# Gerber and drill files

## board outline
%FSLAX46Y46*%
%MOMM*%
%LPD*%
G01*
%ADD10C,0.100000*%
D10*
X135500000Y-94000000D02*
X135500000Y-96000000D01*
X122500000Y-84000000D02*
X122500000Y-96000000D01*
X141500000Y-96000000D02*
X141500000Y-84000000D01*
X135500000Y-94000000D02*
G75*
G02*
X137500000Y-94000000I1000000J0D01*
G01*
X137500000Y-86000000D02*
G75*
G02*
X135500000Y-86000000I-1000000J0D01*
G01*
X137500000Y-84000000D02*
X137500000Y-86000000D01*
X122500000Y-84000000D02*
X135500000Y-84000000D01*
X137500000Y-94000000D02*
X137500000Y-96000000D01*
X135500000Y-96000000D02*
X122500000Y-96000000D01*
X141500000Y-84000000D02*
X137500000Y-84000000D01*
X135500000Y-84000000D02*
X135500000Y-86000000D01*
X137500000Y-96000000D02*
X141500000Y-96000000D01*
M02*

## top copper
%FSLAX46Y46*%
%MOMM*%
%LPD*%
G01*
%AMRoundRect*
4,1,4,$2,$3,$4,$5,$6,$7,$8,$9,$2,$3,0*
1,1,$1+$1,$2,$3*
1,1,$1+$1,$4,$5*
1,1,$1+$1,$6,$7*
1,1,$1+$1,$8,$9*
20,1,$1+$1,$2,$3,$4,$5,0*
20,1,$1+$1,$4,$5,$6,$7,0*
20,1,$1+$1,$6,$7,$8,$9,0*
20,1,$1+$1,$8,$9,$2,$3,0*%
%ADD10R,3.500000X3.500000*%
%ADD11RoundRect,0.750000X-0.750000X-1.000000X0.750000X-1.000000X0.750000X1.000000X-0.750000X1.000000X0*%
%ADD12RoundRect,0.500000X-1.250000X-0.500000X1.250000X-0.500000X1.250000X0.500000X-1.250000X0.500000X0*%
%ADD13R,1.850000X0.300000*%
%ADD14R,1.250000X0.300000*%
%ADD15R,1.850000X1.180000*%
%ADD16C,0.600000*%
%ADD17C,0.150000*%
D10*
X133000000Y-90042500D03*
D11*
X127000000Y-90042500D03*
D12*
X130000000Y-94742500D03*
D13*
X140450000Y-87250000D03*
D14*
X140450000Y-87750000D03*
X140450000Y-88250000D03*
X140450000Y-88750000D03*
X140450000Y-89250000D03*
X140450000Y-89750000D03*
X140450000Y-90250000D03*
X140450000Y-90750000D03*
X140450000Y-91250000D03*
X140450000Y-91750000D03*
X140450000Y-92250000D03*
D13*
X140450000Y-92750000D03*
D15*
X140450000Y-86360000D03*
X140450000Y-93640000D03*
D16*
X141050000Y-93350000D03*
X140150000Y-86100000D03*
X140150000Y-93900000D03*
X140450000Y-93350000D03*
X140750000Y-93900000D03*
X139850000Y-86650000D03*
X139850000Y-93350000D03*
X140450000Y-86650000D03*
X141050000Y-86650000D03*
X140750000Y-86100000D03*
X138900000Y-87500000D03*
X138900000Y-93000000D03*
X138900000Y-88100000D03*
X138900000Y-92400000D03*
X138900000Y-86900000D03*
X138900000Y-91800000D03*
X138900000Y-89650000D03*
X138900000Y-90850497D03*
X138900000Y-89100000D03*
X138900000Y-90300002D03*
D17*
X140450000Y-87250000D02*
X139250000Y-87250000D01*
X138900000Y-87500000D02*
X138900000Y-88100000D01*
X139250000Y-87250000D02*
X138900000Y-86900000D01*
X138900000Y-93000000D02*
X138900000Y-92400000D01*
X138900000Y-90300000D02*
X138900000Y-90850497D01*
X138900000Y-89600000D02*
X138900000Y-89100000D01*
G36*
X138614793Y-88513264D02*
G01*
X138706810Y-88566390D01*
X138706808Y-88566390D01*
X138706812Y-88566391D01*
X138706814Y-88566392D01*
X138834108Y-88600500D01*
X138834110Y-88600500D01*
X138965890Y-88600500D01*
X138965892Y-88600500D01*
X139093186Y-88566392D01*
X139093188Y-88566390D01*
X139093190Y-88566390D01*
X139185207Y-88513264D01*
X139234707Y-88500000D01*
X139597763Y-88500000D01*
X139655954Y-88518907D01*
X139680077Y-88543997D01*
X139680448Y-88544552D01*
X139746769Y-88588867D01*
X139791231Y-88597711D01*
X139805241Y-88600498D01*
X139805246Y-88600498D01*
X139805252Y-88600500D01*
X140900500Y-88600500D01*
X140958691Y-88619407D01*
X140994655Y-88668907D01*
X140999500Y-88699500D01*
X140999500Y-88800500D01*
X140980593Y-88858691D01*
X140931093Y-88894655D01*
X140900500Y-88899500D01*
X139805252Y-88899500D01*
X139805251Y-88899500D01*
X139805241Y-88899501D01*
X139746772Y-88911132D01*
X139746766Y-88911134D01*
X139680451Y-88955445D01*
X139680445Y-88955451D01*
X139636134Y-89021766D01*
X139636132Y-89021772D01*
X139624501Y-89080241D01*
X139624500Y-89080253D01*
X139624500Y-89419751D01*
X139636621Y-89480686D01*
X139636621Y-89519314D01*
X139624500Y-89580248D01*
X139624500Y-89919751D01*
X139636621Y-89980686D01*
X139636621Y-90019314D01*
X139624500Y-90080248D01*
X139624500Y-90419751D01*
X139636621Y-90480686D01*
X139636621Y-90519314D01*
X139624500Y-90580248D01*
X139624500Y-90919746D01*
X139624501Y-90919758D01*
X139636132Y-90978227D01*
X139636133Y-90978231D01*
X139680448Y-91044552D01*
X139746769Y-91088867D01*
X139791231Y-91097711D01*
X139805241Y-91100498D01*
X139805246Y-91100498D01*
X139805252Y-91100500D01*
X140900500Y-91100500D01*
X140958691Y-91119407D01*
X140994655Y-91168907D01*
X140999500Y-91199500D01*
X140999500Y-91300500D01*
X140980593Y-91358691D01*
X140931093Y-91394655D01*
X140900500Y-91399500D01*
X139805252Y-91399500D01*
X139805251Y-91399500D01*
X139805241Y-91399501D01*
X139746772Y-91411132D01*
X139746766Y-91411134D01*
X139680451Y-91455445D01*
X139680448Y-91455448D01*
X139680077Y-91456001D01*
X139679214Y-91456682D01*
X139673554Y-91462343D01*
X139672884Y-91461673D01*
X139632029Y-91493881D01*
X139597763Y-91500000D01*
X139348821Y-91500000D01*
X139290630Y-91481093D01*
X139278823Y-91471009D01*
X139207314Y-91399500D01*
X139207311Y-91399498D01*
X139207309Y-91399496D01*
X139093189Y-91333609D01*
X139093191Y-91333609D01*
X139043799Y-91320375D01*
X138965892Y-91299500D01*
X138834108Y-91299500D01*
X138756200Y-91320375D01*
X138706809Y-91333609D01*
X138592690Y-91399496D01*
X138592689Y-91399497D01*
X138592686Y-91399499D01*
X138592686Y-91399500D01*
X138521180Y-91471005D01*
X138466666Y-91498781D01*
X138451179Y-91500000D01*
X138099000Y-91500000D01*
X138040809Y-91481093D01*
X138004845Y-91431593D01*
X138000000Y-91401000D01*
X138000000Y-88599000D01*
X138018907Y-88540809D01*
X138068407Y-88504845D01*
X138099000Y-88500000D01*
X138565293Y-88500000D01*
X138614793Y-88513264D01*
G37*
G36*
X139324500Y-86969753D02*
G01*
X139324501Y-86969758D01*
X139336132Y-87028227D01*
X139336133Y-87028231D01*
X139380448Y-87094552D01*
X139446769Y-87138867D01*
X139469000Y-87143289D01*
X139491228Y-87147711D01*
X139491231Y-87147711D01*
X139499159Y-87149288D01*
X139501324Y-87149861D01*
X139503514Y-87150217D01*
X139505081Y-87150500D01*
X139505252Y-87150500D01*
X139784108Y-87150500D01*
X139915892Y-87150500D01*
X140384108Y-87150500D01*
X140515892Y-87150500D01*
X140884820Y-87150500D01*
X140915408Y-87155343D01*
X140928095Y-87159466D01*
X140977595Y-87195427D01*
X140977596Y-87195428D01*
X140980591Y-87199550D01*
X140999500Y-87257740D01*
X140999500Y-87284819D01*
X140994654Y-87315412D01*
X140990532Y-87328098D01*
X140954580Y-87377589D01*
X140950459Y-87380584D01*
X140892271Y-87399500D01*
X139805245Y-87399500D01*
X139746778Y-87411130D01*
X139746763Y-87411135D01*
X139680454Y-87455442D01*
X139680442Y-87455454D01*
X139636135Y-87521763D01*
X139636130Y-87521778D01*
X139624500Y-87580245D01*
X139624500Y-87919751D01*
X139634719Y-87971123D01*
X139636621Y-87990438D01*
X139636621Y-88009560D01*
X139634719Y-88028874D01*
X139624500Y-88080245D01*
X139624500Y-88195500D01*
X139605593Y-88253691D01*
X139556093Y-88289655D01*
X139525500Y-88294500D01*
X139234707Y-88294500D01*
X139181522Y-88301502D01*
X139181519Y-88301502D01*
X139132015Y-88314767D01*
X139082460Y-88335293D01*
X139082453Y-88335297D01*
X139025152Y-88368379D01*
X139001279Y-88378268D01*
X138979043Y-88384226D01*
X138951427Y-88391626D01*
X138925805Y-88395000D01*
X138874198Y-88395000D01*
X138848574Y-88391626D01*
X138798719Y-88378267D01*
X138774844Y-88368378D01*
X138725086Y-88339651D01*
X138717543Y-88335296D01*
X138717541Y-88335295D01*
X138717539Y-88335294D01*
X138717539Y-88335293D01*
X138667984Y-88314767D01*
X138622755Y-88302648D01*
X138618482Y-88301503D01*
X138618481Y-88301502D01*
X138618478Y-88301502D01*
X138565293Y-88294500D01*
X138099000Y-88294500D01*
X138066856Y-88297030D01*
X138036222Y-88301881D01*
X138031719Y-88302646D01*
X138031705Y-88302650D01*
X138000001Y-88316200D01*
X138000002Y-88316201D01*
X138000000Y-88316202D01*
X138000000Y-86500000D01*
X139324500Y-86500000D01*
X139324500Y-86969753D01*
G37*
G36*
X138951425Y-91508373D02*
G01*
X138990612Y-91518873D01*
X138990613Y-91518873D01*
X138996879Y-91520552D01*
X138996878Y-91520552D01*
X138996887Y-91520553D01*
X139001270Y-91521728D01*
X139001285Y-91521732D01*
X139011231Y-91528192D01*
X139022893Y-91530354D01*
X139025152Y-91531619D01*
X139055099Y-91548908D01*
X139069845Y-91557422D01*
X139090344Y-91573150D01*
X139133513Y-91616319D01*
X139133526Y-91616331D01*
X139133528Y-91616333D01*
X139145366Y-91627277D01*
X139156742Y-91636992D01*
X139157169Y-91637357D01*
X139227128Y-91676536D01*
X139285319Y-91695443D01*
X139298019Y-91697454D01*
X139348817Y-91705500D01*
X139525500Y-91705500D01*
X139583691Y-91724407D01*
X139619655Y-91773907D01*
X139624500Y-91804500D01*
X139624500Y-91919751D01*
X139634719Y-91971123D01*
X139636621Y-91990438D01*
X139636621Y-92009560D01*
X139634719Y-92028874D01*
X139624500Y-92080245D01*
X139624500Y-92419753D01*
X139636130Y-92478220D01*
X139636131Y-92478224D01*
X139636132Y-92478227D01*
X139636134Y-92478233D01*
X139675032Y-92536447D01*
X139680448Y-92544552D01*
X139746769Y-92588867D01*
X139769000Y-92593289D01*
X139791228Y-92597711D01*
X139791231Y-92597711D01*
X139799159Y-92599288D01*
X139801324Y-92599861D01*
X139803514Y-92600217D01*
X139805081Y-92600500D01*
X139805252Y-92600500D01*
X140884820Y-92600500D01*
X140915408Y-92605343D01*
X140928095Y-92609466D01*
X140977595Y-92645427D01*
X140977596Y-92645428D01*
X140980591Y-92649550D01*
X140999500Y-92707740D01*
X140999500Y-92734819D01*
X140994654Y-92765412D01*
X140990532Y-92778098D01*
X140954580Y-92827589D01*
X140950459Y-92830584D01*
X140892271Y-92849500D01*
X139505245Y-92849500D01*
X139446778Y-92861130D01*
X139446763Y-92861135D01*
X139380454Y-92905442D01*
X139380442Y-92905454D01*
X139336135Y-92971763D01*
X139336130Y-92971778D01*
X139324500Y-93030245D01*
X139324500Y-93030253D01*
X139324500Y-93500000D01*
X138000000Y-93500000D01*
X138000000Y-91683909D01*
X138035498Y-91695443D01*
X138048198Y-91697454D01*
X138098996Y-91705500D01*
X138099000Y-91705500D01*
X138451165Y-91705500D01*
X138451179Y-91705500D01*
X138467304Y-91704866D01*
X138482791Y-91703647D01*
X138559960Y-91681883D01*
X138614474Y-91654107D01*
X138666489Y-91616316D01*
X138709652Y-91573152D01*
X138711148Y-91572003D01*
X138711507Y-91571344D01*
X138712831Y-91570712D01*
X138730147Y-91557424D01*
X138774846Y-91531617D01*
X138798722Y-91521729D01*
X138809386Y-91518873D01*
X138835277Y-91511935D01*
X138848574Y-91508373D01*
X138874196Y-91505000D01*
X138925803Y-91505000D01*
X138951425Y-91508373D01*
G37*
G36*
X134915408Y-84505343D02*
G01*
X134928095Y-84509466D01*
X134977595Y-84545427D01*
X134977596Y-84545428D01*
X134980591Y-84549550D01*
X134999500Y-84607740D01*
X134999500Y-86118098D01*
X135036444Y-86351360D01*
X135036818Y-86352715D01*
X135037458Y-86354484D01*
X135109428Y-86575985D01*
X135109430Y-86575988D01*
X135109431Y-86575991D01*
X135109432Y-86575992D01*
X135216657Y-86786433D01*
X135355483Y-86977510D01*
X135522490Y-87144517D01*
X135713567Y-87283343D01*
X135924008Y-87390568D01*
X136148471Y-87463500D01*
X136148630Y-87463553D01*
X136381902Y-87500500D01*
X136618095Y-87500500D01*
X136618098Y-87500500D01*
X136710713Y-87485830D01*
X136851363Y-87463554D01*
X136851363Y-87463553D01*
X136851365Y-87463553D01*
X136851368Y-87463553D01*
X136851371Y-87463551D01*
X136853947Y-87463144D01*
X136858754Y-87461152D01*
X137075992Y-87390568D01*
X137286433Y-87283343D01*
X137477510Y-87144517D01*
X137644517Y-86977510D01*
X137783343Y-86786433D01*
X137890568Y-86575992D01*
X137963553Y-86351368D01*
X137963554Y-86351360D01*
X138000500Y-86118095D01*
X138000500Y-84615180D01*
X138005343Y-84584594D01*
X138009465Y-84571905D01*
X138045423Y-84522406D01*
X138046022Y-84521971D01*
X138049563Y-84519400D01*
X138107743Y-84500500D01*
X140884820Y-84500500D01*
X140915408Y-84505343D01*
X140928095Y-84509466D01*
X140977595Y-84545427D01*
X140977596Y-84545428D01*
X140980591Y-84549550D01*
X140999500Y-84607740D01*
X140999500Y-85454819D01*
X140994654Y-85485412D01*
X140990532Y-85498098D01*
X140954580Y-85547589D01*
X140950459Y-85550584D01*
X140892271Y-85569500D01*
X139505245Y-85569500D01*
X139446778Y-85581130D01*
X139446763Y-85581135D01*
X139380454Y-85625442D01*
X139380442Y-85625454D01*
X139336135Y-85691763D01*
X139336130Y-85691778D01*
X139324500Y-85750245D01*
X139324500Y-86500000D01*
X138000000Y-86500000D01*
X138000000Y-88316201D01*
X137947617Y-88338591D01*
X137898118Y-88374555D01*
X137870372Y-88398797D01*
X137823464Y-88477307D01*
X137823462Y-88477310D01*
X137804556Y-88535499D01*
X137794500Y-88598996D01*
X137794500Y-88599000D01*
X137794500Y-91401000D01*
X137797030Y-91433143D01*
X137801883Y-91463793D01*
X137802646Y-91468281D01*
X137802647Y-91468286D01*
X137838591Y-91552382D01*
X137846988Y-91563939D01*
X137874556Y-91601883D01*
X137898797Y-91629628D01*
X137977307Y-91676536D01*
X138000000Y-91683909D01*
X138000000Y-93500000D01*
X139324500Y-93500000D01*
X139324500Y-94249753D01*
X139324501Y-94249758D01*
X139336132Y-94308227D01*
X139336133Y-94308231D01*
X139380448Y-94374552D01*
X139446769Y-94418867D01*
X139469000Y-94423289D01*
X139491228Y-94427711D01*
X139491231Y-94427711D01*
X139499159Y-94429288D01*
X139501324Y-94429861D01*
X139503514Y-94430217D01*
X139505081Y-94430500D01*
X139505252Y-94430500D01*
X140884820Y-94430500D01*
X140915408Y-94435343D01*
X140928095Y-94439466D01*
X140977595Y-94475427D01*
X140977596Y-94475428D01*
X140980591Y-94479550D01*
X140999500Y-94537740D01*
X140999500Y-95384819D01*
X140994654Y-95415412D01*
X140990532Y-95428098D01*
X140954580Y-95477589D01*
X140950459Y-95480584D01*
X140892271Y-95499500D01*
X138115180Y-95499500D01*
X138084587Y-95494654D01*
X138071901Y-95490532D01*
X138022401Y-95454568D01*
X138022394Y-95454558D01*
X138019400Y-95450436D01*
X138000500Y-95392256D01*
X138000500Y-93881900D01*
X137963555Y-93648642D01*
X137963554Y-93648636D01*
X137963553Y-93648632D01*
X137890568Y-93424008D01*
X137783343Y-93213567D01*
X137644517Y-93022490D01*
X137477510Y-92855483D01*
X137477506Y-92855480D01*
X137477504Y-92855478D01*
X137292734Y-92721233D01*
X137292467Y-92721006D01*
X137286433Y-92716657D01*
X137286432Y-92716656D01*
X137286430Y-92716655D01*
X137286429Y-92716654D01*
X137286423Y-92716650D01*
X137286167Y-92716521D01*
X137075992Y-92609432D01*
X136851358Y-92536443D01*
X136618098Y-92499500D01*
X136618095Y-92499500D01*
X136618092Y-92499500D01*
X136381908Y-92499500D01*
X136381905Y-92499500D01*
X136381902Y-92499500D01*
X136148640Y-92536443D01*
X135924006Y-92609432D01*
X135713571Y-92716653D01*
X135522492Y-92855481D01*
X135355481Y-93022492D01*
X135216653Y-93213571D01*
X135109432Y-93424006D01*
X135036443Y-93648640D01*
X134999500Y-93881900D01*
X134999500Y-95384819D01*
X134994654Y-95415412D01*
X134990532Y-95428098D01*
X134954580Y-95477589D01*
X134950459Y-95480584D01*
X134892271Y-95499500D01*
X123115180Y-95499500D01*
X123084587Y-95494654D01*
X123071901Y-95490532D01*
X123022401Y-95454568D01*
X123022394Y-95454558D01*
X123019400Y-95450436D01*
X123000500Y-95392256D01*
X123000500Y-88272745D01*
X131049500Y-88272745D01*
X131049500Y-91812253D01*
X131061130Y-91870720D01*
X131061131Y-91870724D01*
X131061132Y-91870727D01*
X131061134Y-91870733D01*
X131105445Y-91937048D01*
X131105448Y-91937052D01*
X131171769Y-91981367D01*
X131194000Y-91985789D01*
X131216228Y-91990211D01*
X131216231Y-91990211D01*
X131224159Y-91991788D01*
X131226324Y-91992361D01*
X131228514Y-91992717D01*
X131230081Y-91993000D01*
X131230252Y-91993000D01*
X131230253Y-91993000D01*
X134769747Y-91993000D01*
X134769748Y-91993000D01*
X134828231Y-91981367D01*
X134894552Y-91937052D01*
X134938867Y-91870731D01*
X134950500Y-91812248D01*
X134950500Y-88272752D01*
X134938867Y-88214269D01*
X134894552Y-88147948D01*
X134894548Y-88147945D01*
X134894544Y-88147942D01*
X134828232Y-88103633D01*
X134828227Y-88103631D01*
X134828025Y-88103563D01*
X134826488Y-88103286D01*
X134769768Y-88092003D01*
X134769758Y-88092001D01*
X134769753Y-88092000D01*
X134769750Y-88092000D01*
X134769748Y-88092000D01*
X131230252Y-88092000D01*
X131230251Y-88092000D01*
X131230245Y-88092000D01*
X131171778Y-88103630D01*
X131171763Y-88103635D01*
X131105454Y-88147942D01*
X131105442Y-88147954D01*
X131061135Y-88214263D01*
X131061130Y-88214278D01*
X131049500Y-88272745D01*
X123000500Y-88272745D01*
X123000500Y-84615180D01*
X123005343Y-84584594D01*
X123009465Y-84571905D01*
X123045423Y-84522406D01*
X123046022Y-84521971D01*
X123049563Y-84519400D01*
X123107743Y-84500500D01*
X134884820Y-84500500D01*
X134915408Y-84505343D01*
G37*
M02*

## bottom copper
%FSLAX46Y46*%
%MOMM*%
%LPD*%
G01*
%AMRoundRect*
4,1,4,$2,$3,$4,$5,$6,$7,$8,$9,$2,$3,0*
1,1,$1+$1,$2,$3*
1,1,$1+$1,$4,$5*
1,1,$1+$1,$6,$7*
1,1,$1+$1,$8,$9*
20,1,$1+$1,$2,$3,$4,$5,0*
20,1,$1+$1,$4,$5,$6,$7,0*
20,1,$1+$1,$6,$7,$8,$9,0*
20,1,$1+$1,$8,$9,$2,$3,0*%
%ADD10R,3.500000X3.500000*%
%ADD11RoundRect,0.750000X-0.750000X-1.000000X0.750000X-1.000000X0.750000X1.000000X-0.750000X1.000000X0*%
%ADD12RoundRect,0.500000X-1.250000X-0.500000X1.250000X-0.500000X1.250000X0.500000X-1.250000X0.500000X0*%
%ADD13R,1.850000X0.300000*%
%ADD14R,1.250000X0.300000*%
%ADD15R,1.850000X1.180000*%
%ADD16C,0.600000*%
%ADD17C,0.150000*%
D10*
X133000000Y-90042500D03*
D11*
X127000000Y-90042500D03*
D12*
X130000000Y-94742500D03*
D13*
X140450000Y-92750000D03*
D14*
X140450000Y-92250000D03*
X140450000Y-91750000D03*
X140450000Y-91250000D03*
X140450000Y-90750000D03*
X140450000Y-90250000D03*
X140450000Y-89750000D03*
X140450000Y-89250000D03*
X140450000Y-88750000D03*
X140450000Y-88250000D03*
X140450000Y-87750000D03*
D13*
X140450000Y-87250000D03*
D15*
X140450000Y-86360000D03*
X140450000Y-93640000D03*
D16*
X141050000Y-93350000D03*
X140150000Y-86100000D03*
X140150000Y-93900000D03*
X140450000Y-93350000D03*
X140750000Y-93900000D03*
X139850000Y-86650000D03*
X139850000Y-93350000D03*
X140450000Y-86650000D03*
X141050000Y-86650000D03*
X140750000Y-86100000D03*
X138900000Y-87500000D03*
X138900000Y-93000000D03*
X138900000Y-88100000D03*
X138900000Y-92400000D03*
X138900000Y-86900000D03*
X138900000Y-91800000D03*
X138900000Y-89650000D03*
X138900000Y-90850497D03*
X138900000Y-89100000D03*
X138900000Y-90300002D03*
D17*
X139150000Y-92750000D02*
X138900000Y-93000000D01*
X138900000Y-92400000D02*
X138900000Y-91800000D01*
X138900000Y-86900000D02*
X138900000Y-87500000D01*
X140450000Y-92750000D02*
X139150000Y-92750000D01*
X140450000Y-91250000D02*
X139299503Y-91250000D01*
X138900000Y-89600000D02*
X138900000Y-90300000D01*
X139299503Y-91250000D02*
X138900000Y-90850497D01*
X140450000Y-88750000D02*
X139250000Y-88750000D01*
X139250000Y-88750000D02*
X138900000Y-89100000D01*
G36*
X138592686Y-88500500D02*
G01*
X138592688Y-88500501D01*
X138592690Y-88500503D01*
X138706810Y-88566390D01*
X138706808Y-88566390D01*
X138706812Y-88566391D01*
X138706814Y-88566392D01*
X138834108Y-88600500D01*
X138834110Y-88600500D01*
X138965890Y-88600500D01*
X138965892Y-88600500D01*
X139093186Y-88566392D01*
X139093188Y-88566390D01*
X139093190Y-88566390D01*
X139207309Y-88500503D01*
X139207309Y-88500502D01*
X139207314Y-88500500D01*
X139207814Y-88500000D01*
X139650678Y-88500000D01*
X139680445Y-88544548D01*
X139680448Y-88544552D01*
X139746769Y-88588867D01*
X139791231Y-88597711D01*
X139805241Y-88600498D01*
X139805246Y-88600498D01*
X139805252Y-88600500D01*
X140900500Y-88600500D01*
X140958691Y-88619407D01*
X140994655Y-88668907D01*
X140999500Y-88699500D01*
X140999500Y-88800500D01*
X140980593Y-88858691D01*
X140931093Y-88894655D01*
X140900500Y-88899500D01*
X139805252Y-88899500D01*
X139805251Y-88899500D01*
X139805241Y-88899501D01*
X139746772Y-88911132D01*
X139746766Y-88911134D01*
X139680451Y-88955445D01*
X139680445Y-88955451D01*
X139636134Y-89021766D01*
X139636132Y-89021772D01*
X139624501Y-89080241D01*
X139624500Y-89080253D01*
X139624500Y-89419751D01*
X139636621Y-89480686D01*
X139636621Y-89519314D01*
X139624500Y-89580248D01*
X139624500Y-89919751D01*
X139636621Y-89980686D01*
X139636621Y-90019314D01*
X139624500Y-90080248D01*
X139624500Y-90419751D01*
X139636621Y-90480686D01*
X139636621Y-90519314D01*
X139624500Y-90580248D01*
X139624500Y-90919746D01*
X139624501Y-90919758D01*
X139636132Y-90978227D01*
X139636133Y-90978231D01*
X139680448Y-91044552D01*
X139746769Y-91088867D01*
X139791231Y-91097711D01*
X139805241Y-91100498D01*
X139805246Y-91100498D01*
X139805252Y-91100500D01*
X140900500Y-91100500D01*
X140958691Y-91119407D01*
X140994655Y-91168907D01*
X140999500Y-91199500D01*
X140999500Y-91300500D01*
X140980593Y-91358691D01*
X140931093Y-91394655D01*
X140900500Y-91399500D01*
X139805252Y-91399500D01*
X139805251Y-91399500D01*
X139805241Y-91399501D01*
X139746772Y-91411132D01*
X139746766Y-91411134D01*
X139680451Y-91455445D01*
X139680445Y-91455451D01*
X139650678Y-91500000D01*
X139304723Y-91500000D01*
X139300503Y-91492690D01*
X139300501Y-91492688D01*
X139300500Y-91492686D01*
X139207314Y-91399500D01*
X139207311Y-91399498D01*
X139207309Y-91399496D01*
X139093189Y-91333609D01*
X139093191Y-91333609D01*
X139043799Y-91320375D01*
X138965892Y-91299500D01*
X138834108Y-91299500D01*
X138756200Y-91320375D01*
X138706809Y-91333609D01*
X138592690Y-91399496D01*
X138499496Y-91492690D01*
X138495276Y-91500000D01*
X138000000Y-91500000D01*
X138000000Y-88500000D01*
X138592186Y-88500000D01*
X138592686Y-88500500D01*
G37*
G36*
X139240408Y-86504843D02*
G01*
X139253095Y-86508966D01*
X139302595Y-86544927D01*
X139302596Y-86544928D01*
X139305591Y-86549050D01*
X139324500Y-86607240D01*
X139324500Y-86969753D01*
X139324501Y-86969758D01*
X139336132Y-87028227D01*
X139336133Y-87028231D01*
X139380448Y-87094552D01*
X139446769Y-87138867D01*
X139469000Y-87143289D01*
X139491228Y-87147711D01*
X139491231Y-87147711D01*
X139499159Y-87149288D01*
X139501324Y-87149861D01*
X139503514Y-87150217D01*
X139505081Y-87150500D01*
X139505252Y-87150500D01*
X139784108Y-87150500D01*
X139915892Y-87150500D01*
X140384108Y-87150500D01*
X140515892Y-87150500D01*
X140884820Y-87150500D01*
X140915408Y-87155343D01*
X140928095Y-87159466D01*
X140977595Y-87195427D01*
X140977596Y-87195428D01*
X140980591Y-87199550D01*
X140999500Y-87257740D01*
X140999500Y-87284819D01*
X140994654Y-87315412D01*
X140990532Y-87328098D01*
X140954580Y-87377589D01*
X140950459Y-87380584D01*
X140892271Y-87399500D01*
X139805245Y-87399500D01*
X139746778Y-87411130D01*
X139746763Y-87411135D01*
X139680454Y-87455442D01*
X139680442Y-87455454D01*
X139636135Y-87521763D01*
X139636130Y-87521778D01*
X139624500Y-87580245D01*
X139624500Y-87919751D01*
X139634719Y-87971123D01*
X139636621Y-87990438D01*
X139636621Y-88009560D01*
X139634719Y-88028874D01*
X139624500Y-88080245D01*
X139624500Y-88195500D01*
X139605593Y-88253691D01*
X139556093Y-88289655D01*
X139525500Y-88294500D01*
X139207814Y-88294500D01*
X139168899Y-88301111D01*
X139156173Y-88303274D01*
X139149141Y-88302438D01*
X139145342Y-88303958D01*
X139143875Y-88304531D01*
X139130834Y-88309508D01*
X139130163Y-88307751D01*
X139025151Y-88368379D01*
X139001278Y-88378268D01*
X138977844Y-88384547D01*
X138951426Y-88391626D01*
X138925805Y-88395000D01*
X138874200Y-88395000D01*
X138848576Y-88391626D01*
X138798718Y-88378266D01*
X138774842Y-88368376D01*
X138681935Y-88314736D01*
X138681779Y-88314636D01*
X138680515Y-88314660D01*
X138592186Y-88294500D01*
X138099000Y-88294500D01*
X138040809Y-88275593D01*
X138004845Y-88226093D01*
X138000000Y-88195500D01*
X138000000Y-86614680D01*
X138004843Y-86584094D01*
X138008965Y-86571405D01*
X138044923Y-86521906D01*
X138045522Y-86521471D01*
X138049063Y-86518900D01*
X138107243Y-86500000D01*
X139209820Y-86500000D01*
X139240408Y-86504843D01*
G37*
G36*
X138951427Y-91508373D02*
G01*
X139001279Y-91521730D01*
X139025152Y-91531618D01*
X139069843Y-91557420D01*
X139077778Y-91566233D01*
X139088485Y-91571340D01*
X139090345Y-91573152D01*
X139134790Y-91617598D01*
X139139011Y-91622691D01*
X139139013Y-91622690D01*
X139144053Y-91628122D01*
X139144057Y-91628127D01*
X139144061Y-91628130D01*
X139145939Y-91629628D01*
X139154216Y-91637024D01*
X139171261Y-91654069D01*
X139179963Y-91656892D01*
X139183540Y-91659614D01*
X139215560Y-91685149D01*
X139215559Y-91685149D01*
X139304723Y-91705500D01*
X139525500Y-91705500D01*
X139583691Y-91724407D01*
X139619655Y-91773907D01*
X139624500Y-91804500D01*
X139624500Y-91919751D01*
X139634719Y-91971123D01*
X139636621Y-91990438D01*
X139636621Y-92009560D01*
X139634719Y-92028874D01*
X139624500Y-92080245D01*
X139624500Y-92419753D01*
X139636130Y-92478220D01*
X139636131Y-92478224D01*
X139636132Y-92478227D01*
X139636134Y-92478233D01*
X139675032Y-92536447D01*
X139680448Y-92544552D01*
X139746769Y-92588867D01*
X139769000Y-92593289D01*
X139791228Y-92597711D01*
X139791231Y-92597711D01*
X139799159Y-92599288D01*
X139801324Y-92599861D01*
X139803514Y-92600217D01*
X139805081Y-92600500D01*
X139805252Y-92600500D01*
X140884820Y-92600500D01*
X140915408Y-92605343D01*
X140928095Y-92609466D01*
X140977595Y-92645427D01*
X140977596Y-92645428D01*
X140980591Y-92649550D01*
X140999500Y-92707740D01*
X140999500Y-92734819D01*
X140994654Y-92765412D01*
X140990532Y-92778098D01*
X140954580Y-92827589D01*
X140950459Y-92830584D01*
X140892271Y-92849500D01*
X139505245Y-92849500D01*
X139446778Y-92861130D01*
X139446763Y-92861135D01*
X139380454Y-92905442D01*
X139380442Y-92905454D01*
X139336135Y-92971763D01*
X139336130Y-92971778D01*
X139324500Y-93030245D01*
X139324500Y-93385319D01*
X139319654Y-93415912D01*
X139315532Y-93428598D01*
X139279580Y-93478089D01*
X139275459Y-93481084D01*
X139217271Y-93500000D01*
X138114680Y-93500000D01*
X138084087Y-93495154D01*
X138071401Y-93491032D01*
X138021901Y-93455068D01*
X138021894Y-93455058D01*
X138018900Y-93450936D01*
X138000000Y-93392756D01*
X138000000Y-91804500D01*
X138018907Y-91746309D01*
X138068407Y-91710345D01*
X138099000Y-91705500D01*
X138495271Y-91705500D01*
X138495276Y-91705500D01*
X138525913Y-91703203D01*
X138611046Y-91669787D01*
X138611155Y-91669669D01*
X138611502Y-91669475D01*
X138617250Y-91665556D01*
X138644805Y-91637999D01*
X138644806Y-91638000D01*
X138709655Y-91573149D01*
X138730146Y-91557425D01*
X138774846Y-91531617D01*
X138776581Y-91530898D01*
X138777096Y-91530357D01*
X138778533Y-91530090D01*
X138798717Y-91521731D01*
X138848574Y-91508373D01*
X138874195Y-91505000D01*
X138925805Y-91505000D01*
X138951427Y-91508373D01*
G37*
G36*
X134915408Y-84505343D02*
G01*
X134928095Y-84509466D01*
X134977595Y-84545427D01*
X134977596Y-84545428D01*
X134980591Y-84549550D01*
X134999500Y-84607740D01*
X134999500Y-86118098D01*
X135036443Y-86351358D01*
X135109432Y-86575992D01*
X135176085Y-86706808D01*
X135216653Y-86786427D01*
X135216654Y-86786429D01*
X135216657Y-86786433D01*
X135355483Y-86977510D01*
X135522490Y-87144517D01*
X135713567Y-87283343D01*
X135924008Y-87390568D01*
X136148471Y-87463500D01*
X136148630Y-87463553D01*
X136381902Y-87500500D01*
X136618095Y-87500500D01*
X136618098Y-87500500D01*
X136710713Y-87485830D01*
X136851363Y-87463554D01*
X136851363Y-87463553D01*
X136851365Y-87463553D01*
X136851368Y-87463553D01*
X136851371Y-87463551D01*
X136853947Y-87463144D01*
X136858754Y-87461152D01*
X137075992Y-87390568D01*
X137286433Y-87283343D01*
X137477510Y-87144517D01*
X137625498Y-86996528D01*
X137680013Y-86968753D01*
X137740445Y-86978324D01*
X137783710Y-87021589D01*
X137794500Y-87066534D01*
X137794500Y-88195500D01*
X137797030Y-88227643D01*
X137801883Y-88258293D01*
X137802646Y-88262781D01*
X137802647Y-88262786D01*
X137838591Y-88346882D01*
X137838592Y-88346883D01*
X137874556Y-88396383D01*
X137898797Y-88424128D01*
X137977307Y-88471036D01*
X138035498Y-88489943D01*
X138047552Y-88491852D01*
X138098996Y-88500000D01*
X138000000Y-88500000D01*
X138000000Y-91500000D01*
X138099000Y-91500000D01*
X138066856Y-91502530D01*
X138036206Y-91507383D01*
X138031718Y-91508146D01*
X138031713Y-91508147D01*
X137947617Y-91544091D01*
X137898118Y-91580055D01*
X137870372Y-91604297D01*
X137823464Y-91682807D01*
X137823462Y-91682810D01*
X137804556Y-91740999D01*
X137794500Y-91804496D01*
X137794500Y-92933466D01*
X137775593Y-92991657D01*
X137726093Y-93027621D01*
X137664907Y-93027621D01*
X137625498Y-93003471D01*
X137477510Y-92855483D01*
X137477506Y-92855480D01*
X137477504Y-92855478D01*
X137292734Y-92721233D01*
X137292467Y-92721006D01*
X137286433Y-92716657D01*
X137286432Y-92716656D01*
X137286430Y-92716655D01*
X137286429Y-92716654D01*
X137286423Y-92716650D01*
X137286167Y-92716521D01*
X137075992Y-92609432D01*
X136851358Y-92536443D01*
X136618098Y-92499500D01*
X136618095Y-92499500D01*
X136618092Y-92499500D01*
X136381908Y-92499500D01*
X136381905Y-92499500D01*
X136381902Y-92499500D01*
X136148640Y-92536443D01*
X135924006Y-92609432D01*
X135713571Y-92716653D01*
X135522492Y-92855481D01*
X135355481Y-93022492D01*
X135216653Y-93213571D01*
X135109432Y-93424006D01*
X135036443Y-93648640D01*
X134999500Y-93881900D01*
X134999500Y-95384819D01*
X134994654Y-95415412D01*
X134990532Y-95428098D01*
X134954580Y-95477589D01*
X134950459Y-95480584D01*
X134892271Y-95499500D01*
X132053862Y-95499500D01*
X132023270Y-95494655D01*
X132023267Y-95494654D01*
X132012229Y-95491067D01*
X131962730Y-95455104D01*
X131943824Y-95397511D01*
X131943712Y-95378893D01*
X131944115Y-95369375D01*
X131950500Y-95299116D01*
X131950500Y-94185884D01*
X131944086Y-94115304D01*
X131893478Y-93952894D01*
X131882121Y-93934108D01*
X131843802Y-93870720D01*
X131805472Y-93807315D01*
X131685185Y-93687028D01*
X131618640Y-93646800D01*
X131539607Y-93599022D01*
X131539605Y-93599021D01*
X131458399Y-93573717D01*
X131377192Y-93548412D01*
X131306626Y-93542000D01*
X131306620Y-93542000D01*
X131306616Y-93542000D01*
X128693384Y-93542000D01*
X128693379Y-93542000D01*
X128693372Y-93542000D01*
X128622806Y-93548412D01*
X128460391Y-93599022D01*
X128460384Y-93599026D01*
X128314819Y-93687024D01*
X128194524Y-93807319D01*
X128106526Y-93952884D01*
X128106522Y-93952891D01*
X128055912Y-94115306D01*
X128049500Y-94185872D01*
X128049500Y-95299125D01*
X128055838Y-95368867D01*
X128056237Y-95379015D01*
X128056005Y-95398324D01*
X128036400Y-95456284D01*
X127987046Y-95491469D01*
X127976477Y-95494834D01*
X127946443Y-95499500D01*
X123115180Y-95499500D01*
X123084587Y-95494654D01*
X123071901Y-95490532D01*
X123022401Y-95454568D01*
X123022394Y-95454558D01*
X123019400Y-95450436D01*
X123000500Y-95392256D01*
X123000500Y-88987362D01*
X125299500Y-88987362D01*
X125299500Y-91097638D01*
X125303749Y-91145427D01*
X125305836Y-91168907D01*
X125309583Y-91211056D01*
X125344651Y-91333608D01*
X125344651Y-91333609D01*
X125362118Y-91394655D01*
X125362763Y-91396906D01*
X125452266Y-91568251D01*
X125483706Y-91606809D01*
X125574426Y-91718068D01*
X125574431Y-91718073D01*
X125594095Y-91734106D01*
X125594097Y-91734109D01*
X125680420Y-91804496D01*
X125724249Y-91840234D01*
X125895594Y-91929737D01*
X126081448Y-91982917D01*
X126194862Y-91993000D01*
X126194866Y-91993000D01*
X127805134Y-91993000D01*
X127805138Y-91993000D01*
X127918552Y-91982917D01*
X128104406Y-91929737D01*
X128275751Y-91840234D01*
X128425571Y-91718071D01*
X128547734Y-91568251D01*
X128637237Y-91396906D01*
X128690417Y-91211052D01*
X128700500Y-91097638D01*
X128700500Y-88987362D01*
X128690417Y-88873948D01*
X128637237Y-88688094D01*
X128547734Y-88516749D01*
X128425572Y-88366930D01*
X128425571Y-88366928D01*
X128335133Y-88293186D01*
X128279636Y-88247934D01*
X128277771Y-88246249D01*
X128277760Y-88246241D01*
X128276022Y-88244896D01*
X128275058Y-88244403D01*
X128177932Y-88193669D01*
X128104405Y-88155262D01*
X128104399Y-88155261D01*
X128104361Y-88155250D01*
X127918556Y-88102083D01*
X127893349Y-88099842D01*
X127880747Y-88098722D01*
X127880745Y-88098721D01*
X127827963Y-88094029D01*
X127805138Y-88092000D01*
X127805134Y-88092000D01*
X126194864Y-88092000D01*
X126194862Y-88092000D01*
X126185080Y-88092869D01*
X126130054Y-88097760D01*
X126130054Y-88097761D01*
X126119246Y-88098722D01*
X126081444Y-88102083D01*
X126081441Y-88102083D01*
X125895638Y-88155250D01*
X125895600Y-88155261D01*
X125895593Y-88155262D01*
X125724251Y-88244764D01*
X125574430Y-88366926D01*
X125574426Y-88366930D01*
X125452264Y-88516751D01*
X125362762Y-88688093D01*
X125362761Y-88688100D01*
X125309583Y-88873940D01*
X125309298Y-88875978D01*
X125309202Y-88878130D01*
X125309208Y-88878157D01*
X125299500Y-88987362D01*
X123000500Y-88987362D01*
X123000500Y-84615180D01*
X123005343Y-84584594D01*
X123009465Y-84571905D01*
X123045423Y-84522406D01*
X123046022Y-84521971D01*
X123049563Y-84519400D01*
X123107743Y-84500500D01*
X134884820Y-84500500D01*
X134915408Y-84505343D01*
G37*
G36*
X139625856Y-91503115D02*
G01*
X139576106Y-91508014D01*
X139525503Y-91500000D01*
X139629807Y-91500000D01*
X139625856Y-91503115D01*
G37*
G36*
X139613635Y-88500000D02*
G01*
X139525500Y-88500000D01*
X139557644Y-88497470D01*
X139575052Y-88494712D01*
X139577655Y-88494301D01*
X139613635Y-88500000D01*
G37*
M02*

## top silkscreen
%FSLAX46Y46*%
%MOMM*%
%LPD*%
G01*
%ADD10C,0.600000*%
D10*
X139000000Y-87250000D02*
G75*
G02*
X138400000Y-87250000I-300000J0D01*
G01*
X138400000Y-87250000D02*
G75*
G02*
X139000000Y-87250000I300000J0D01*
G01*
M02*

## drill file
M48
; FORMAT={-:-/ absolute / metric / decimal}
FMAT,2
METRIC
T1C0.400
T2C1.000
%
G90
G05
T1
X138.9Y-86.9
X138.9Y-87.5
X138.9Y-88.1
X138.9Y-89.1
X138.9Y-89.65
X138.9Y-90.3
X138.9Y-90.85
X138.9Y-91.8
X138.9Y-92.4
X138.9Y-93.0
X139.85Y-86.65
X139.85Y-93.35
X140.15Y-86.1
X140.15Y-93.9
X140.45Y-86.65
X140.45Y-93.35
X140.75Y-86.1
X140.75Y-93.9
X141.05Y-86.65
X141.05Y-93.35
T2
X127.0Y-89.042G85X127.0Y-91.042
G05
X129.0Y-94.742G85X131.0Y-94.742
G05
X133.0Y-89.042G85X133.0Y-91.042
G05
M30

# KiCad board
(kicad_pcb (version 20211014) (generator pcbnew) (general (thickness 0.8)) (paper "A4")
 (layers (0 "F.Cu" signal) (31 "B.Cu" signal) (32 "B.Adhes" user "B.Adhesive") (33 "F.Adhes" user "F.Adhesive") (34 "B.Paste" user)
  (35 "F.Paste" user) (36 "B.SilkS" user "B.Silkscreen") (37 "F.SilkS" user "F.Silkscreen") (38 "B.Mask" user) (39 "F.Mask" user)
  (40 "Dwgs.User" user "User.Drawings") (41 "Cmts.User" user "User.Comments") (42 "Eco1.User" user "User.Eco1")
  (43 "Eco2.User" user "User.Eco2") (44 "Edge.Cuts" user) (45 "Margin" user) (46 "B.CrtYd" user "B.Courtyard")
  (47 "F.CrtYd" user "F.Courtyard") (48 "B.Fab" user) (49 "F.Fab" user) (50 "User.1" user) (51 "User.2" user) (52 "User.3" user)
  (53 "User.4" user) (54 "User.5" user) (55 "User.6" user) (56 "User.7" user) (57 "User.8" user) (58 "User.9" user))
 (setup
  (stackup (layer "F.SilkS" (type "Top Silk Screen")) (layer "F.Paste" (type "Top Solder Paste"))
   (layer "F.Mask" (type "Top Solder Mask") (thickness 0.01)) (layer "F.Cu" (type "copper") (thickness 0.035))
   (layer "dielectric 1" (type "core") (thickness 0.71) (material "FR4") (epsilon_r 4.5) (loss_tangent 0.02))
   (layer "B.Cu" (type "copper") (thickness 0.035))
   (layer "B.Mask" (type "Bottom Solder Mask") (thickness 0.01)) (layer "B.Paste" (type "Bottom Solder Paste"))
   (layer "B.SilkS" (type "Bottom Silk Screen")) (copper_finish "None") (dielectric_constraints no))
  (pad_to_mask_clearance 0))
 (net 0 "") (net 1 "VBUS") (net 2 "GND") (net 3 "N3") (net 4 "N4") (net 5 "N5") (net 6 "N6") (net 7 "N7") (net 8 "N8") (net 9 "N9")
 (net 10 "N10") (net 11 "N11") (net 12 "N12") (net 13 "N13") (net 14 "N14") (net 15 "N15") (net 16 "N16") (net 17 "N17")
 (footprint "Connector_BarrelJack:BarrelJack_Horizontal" (layer "F.Cu") (at 133 90.0425)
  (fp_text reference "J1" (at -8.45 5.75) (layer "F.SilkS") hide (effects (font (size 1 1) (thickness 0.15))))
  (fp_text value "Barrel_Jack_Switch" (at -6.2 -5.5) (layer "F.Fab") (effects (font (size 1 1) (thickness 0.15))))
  (pad "1" thru_hole rect (at 0 0) (size 3.5 3.5) (drill oval 1 3) (layers *.Cu *.Mask) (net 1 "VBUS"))
  (pad "2" thru_hole roundrect (at -6 0) (size 3 3.5) (drill oval 1 3) (layers *.Cu *.Mask) (roundrect_rratio 0.25) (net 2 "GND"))
  (pad "3" thru_hole roundrect (at -3 4.7) (size 3.5 2) (drill oval 3 1) (layers *.Cu *.Mask) (roundrect_rratio 0.25) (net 2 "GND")))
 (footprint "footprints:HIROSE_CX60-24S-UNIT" (layer "F.Cu") (at 140.45 90 90)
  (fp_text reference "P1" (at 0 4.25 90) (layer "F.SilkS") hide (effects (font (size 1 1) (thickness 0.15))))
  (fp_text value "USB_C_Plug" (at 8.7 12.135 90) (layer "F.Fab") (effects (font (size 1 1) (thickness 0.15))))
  (fp_circle (center 2.75 -1.75) (end 3.25 -1.75) (layer "F.SilkS") (width 0.2) (fill solid))
  (pad "A1" smd rect (at 2.75 0 90) (size 0.3 1.85) (layers "F.Cu" "F.Paste" "F.Mask") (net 2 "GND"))
  (pad "A2" smd rect (at 2.25 0 90) (size 0.3 1.25) (layers "F.Cu" "F.Paste" "F.Mask") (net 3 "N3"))
  (pad "A3" smd rect (at 1.75 0 90) (size 0.3 1.25) (layers "F.Cu" "F.Paste" "F.Mask") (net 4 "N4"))
  (pad "A4" smd rect (at 1.25 0 90) (size 0.3 1.25) (layers "F.Cu" "F.Paste" "F.Mask") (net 1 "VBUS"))
  (pad "A5" smd rect (at 0.75 0 90) (size 0.3 1.25) (layers "F.Cu" "F.Paste" "F.Mask") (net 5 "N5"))
  (pad "A6" smd rect (at 0.25 0 90) (size 0.3 1.25) (layers "F.Cu" "F.Paste" "F.Mask") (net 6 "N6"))
  (pad "A7" smd rect (at -0.25 0 90) (size 0.3 1.25) (layers "F.Cu" "F.Paste" "F.Mask") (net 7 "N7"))
  (pad "A8" smd rect (at -0.75 0 90) (size 0.3 1.25) (layers "F.Cu" "F.Paste" "F.Mask") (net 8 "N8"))
  (pad "A9" smd rect (at -1.25 0 90) (size 0.3 1.25) (layers "F.Cu" "F.Paste" "F.Mask") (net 1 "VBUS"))
  (pad "A10" smd rect (at -1.75 0 90) (size 0.3 1.25) (layers "F.Cu" "F.Paste" "F.Mask") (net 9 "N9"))
  (pad "A11" smd rect (at -2.25 0 90) (size 0.3 1.25) (layers "F.Cu" "F.Paste" "F.Mask") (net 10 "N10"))
  (pad "A12" smd rect (at -2.75 0 90) (size 0.3 1.85) (layers "F.Cu" "F.Paste" "F.Mask") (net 2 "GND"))
  (pad "B1" smd rect (at -2.75 0 90) (size 0.3 1.85) (layers "B.Cu" "B.Paste" "B.Mask") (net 2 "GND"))
  (pad "B2" smd rect (at -2.25 0 90) (size 0.3 1.25) (layers "B.Cu" "B.Paste" "B.Mask") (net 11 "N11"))
  (pad "B3" smd rect (at -1.75 0 90) (size 0.3 1.25) (layers "B.Cu" "B.Paste" "B.Mask") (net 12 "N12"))
  (pad "B4" smd rect (at -1.25 0 90) (size 0.3 1.25) (layers "B.Cu" "B.Paste" "B.Mask") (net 1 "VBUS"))
  (pad "B5" smd rect (at -0.75 0 90) (size 0.3 1.25) (layers "B.Cu" "B.Paste" "B.Mask") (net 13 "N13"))
  (pad "B6" smd rect (at -0.25 0 90) (size 0.3 1.25) (layers "B.Cu" "B.Paste" "B.Mask"))
  (pad "B7" smd rect (at 0.25 0 90) (size 0.3 1.25) (layers "B.Cu" "B.Paste" "B.Mask"))
  (pad "B8" smd rect (at 0.75 0 90) (size 0.3 1.25) (layers "B.Cu" "B.Paste" "B.Mask") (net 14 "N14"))
  (pad "B9" smd rect (at 1.25 0 90) (size 0.3 1.25) (layers "B.Cu" "B.Paste" "B.Mask") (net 1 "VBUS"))
  (pad "B10" smd rect (at 1.75 0 90) (size 0.3 1.25) (layers "B.Cu" "B.Paste" "B.Mask") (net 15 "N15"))
  (pad "B11" smd rect (at 2.25 0 90) (size 0.3 1.25) (layers "B.Cu" "B.Paste" "B.Mask") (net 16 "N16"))
  (pad "B12" smd rect (at 2.75 0 90) (size 0.3 1.85) (layers "B.Cu" "B.Paste" "B.Mask") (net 2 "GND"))
  (pad "S1" smd rect (at 3.64 0 90) (size 1.18 1.85) (layers "F.Cu" "F.Paste" "F.Mask") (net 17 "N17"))
  (pad "S2" smd rect (at -3.64 0 90) (size 1.18 1.85) (layers "F.Cu" "F.Paste" "F.Mask"))
  (pad "S3" smd rect (at 3.64 0 90) (size 1.18 1.85) (layers "B.Cu" "B.Paste" "B.Mask"))
  (pad "S4" smd rect (at -3.64 0 90) (size 1.18 1.85) (layers "B.Cu" "B.Paste" "B.Mask")))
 (gr_line (start 135.5 94) (end 135.5 96) (layer "Edge.Cuts") (width 0.1))
 (gr_line (start 122.5 84) (end 122.5 96) (layer "Edge.Cuts") (width 0.1))
 (gr_line (start 141.5 96) (end 141.5 84) (layer "Edge.Cuts") (width 0.1))
 (gr_arc locked (start 135.5 94) (mid 136.5 93) (end 137.5 94) (layer "Edge.Cuts") (width 0.1))
 (gr_arc locked (start 137.5 86) (mid 136.5 87) (end 135.5 86) (layer "Edge.Cuts") (width 0.1))
 (gr_line (start 137.5 84) (end 137.5 86) (layer "Edge.Cuts") (width 0.1))
 (gr_line (start 122.5 84) (end 135.5 84) (layer "Edge.Cuts") (width 0.1))
 (gr_line (start 137.5 94) (end 137.5 96) (layer "Edge.Cuts") (width 0.1))
 (gr_line (start 135.5 96) (end 122.5 96) (layer "Edge.Cuts") (width 0.1))
 (gr_line (start 141.5 84) (end 137.5 84) (layer "Edge.Cuts") (width 0.1))
 (gr_line (start 135.5 84) (end 135.5 86) (layer "Edge.Cuts") (width 0.1))
 (gr_line (start 137.5 96) (end 141.5 96) (layer "Edge.Cuts") (width 0.1))
 (via (at 141.05 93.35) (size 0.6) (drill 0.4) (layers "F.Cu" "B.Cu") (free) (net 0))
 (via (at 140.15 86.1) (size 0.6) (drill 0.4) (layers "F.Cu" "B.Cu") (free) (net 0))
 (via (at 140.15 93.9) (size 0.6) (drill 0.4) (layers "F.Cu" "B.Cu") (free) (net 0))
 (via (at 140.45 93.35) (size 0.6) (drill 0.4) (layers "F.Cu" "B.Cu") (free) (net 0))
 (via (at 140.75 93.9) (size 0.6) (drill 0.4) (layers "F.Cu" "B.Cu") (free) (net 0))
 (via (at 139.85 86.65) (size 0.6) (drill 0.4) (layers "F.Cu" "B.Cu") (free) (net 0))
 (via (at 139.85 93.35) (size 0.6) (drill 0.4) (layers "F.Cu" "B.Cu") (free) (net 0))
 (via (at 140.45 86.65) (size 0.6) (drill 0.4) (layers "F.Cu" "B.Cu") (free) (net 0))
 (via (at 141.05 86.65) (size 0.6) (drill 0.4) (layers "F.Cu" "B.Cu") (free) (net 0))
 (via (at 140.75 86.1) (size 0.6) (drill 0.4) (layers "F.Cu" "B.Cu") (free) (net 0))
 (segment (start 140.45 87.25) (end 139.25 87.25) (width 0.15) (layer "F.Cu") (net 2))
 (segment (start 138.9 87.5) (end 138.9 88.1) (width 0.15) (layer "F.Cu") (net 2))
 (segment (start 139.25 87.25) (end 138.9 86.9) (width 0.15) (layer "F.Cu") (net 2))
 (segment (start 138.9 93) (end 138.9 92.4) (width 0.15) (layer "F.Cu") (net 2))
 (via (at 138.9 87.5) (size 0.6) (drill 0.4) (layers "F.Cu" "B.Cu") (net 2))
 (via (at 138.9 93) (size 0.6) (drill 0.4) (layers "F.Cu" "B.Cu") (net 2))
 (via (at 138.9 88.1) (size 0.6) (drill 0.4) (layers "F.Cu" "B.Cu") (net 2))
 (via (at 138.9 92.4) (size 0.6) (drill 0.4) (layers "F.Cu" "B.Cu") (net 2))
 (via (at 138.9 86.9) (size 0.6) (drill 0.4) (layers "F.Cu" "B.Cu") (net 2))
 (via (at 138.9 91.8) (size 0.6) (drill 0.4) (layers "F.Cu" "B.Cu") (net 2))
 (segment (start 139.15 92.75) (end 138.9 93) (width 0.15) (layer "B.Cu") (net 2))
 (segment (start 138.9 92.4) (end 138.9 91.8) (width 0.15) (layer "B.Cu") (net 2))
 (segment (start 138.9 86.9) (end 138.9 87.5) (width 0.15) (layer "B.Cu") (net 2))
 (segment (start 140.45 92.75) (end 139.15 92.75) (width 0.15) (layer "B.Cu") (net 2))
 (segment (start 138.9 90.3) (end 138.9 90.850497) (width 0.15) (layer "F.Cu") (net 1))
 (segment (start 138.9 89.6) (end 138.9 89.1) (width 0.15) (layer "F.Cu") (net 1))
 (via (at 138.9 89.65) (size 0.6) (drill 0.4) (layers "F.Cu" "B.Cu") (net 1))
 (via (at 138.9 90.850497) (size 0.6) (drill 0.4) (layers "F.Cu" "B.Cu") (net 1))
 (via (at 138.9 89.1) (size 0.6) (drill 0.4) (layers "F.Cu" "B.Cu") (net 1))
 (via (at 138.9 90.300002) (size 0.6) (drill 0.4) (layers "F.Cu" "B.Cu") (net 1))
 (segment (start 140.45 91.25) (end 139.299503 91.25) (width 0.15) (layer "B.Cu") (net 1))
 (segment (start 138.9 89.6) (end 138.9 90.3) (width 0.15) (layer "B.Cu") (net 1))
 (segment (start 139.299503 91.25) (end 138.9 90.850497) (width 0.15) (layer "B.Cu") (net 1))
 (segment (start 140.45 88.75) (end 139.25 88.75) (width 0.15) (layer "B.Cu") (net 1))
 (segment (start 139.25 88.75) (end 138.9 89.1) (width 0.15) (layer "B.Cu") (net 1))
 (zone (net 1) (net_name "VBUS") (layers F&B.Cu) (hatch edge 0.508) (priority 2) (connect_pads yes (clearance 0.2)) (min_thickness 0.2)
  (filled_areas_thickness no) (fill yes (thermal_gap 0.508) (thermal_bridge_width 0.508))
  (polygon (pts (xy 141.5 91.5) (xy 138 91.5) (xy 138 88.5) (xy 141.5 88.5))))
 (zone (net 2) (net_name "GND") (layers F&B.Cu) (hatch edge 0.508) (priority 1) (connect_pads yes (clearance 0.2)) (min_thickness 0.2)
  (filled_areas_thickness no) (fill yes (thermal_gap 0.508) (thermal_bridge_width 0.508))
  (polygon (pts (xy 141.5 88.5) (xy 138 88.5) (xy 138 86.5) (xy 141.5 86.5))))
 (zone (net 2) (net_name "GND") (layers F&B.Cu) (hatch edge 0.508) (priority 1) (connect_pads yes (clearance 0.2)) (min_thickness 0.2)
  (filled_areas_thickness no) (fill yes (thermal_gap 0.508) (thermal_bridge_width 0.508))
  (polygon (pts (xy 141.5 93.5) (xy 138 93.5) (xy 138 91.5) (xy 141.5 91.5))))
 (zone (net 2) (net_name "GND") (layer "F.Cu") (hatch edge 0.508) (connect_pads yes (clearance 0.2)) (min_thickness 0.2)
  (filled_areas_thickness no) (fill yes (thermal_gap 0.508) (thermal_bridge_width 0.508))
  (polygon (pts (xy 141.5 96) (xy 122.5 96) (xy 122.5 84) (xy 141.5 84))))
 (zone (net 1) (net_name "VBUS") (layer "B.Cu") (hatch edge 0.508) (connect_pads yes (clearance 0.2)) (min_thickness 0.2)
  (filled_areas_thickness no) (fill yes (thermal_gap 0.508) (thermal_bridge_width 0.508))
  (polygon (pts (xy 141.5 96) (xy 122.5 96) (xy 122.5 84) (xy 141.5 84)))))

